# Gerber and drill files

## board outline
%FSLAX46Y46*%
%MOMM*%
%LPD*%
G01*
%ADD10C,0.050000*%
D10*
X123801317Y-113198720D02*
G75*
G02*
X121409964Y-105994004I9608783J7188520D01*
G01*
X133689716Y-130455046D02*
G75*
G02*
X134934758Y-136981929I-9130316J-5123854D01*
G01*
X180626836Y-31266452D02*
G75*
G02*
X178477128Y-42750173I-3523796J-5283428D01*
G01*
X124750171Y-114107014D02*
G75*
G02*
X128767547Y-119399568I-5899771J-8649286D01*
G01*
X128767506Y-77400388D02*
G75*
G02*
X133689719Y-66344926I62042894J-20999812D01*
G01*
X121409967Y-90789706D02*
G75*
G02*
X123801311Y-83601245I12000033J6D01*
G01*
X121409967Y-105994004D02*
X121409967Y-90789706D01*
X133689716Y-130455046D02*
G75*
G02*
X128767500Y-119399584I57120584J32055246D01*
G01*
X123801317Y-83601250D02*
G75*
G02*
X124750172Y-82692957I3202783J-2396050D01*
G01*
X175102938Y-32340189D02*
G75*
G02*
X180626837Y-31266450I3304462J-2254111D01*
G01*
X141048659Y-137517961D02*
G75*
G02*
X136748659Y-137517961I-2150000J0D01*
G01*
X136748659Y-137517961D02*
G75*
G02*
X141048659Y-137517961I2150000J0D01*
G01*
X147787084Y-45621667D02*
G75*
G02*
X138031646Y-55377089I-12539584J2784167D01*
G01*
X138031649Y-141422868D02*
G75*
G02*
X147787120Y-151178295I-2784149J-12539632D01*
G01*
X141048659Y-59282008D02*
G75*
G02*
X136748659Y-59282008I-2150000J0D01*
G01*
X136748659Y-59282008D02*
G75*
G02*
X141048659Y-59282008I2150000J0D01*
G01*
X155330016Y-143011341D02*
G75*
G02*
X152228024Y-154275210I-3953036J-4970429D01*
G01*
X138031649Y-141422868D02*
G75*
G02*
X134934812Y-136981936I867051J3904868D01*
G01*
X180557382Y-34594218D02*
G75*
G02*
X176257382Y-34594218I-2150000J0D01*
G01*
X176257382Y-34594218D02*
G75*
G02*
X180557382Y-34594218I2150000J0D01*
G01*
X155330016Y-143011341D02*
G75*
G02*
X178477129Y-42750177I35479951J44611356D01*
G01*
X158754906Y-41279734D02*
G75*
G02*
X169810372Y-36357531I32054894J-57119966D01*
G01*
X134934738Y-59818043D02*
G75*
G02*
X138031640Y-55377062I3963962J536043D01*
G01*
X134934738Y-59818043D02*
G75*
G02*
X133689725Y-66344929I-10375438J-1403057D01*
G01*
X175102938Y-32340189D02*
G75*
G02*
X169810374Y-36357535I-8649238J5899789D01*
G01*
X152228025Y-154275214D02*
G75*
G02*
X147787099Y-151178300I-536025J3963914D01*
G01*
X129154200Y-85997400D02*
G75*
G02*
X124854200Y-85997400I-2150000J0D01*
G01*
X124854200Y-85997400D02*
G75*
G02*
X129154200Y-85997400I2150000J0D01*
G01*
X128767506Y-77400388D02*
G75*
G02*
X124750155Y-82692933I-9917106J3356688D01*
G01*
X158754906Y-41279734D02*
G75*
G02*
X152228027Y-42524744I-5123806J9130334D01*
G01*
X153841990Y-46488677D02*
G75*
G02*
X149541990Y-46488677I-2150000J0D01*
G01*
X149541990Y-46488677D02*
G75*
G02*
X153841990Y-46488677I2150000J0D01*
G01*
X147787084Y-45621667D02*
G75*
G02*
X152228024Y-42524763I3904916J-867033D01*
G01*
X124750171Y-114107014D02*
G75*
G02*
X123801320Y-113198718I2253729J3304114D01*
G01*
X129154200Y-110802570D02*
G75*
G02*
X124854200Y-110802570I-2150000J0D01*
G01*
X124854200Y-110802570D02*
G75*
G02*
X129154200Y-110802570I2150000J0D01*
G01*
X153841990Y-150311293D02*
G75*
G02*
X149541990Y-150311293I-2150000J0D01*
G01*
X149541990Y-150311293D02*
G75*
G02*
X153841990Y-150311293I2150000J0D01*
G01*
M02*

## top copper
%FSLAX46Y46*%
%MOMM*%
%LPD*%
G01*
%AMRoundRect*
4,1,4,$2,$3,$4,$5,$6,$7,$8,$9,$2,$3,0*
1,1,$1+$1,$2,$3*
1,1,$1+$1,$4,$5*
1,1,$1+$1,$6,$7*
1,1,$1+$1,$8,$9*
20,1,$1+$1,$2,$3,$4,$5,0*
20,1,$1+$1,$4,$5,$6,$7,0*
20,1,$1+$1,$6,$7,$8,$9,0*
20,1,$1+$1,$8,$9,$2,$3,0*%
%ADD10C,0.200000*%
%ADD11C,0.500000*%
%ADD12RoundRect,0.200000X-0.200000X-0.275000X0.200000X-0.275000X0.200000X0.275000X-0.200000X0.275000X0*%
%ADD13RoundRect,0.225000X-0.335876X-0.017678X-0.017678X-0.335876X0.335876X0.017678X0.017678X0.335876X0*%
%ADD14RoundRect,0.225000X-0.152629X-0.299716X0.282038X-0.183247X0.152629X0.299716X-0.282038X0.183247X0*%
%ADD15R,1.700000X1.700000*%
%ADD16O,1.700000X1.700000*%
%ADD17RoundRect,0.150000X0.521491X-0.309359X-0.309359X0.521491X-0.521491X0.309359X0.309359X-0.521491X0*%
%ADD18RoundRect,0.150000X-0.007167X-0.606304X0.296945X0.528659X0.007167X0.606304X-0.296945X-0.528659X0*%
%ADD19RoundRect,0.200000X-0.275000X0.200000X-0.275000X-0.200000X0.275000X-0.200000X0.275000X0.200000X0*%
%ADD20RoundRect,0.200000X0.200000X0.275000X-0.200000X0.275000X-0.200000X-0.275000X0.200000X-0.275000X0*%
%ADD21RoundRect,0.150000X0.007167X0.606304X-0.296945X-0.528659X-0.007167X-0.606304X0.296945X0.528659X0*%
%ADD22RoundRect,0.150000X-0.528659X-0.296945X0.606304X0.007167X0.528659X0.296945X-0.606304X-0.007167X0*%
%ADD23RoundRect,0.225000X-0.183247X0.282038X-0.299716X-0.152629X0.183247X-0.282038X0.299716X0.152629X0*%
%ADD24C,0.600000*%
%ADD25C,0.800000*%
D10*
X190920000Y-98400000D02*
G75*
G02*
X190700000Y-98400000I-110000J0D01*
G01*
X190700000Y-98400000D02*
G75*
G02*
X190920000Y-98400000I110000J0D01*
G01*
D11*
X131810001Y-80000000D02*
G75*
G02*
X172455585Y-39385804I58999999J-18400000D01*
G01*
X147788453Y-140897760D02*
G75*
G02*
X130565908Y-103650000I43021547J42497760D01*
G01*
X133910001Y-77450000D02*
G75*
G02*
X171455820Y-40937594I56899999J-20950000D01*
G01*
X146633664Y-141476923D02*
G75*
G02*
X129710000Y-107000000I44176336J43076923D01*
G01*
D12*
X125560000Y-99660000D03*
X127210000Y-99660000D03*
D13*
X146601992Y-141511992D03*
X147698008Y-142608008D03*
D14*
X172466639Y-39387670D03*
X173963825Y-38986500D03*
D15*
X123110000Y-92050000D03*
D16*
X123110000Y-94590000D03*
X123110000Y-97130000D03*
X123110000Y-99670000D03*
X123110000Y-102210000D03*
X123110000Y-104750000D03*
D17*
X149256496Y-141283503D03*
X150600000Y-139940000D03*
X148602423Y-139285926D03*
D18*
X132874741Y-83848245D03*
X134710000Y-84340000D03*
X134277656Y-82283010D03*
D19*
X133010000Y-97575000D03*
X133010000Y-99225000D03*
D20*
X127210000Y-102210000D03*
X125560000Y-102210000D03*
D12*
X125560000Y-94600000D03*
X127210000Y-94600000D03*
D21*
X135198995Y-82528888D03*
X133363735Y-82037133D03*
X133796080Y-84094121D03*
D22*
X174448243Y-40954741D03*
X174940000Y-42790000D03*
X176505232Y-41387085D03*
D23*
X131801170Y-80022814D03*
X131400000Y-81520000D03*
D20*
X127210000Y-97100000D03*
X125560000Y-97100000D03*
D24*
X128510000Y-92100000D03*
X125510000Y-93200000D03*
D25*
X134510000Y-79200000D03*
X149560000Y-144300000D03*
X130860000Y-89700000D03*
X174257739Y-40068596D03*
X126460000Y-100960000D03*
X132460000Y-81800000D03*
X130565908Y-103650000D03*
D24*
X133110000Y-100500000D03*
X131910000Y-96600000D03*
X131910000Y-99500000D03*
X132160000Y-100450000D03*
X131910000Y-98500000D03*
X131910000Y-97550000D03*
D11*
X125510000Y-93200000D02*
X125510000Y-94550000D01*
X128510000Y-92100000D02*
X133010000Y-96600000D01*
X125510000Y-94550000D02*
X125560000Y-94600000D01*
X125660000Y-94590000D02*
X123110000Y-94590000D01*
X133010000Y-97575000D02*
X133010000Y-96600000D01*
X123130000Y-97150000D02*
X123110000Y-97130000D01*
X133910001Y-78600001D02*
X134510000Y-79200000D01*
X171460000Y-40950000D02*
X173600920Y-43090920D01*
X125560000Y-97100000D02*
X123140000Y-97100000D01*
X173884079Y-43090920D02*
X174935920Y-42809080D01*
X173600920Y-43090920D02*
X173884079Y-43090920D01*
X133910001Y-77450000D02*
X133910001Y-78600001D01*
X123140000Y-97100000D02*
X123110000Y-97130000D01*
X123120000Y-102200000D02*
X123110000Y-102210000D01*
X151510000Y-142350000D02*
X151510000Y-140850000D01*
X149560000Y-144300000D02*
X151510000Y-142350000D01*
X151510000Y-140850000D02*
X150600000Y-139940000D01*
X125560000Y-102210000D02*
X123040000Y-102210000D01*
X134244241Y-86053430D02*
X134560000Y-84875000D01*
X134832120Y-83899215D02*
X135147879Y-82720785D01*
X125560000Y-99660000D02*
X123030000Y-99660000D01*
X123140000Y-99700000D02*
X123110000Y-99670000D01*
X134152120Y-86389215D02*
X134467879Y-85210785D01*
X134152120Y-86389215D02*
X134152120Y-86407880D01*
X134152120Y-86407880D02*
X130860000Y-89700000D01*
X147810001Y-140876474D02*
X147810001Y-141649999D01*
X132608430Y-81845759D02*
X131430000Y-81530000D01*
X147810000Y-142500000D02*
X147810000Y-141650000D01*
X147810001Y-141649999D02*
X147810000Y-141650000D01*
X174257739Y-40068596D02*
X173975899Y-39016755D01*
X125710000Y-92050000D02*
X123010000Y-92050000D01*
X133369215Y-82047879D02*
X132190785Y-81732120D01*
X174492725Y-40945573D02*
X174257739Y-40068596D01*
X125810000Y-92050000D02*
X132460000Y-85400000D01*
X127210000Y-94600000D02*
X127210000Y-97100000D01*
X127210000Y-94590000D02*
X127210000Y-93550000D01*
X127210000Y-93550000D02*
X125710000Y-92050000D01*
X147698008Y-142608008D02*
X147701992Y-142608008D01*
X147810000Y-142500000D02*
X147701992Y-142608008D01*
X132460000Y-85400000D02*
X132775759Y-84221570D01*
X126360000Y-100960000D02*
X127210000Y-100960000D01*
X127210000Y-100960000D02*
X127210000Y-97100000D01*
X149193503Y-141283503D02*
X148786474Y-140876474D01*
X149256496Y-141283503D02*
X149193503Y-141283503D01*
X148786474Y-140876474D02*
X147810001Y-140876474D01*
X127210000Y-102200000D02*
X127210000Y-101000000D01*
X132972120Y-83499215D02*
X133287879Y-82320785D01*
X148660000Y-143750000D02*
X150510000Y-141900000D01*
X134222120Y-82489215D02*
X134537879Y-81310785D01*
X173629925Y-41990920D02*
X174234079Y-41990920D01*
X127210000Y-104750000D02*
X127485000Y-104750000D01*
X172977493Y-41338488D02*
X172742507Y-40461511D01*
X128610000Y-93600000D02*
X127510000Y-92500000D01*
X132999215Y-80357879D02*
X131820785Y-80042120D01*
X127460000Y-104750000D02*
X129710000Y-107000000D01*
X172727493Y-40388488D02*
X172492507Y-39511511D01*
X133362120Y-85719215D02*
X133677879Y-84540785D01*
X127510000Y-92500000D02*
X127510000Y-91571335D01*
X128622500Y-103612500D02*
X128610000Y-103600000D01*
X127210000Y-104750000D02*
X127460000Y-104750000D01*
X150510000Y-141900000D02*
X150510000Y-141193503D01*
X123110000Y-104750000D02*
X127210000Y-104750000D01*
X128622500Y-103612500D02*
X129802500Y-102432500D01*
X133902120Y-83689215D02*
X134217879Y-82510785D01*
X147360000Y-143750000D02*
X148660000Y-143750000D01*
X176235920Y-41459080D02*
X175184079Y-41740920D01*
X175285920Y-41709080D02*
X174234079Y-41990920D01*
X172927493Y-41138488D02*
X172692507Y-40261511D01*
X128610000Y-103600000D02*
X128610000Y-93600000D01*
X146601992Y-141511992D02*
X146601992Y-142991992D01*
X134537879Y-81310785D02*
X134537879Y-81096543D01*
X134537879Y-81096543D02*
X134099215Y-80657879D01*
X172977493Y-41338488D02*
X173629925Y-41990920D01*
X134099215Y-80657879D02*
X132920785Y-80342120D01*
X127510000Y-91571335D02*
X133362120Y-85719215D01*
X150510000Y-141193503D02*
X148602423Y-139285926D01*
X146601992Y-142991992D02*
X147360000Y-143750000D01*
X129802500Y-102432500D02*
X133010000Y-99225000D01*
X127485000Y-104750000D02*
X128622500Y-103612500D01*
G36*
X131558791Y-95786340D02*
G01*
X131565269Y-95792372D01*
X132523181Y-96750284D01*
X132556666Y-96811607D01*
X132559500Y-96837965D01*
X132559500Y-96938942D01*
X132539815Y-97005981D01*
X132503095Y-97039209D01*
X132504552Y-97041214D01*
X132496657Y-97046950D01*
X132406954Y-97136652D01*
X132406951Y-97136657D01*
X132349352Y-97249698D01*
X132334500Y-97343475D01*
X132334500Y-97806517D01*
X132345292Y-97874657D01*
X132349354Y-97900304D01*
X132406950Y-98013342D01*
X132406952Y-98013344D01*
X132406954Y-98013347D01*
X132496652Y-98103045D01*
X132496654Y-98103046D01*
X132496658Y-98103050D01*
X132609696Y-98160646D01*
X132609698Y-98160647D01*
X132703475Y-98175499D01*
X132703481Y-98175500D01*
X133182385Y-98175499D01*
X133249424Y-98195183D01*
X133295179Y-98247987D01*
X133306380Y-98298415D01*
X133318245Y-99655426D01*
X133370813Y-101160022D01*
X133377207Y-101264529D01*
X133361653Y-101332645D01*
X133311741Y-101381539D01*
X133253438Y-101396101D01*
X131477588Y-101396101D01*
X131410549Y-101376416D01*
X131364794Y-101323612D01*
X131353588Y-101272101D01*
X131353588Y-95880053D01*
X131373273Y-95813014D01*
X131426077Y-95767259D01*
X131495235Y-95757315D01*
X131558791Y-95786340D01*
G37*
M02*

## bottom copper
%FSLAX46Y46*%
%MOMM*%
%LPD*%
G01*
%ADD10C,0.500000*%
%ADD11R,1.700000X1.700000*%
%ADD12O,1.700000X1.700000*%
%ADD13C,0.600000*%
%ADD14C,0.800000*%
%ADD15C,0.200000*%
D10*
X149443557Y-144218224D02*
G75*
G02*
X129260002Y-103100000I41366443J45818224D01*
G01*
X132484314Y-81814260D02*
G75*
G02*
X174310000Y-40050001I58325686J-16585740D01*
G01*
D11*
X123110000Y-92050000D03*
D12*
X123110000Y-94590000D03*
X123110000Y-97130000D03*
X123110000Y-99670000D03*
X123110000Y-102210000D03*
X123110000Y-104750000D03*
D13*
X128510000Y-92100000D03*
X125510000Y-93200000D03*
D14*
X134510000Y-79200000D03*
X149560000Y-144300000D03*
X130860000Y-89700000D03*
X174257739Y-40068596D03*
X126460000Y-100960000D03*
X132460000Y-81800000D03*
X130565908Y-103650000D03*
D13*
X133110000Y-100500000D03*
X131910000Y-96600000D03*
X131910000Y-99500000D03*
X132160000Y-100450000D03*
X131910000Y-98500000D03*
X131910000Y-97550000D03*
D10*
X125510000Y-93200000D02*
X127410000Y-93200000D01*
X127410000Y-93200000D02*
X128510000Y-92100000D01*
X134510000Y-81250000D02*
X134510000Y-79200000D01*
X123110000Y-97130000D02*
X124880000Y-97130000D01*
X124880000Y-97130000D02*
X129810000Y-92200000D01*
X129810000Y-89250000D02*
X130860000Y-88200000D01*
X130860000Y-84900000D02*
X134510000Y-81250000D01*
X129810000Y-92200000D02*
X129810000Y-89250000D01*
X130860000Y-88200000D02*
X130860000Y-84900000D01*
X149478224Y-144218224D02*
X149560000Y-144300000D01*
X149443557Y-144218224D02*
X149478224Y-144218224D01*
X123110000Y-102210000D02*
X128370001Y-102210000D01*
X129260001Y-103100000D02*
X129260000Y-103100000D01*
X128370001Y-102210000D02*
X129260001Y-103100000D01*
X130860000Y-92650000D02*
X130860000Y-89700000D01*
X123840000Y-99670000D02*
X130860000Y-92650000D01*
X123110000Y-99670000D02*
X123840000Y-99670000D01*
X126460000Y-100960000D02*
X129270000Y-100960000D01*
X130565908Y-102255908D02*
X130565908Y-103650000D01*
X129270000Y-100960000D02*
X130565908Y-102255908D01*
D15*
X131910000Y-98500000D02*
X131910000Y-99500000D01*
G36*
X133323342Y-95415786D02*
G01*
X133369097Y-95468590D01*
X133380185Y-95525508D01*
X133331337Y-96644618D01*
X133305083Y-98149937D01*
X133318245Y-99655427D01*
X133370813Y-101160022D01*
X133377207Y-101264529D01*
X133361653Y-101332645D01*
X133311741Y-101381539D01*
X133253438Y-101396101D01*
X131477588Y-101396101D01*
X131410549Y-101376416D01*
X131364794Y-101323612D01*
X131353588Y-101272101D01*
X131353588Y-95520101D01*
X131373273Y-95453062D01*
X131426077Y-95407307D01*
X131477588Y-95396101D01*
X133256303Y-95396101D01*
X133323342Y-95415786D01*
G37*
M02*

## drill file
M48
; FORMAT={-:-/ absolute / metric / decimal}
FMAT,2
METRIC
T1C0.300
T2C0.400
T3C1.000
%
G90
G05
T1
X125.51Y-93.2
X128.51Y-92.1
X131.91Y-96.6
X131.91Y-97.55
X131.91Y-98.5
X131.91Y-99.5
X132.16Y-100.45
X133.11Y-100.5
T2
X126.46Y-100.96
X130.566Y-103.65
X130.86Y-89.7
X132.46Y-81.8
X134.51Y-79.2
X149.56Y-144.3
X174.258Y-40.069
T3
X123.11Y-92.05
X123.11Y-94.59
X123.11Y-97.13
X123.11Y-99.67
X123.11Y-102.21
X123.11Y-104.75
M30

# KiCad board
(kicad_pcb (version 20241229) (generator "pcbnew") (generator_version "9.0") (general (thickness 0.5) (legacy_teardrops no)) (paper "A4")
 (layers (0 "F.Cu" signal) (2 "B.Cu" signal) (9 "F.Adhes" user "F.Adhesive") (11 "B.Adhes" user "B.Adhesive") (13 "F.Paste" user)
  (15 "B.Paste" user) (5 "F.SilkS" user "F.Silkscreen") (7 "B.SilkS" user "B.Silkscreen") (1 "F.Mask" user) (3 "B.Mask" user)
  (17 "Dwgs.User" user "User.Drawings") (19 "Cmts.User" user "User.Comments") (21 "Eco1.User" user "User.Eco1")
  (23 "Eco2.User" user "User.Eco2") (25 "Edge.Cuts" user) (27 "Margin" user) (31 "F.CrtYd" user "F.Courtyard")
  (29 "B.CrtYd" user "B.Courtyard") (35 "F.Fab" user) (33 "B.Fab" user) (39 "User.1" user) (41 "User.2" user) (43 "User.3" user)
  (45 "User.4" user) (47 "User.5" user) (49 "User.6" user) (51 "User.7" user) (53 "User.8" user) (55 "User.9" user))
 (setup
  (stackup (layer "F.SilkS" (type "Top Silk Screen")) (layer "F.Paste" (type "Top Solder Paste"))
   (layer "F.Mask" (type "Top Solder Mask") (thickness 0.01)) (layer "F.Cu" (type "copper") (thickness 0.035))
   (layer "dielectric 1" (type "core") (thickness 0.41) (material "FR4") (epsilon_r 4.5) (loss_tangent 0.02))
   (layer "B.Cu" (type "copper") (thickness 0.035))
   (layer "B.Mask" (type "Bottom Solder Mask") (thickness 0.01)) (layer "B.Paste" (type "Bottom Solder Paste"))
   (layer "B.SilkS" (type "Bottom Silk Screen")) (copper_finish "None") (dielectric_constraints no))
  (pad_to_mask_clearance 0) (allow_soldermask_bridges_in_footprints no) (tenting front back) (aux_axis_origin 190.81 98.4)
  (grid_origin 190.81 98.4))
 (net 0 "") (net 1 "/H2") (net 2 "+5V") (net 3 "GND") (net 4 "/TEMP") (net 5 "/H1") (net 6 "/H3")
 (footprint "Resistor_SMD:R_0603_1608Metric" (layer "F.Cu") (at 126.385 99.66)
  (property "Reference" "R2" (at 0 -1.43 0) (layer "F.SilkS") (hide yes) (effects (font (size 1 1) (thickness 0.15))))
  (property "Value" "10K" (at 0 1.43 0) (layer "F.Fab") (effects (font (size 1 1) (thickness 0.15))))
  (pad "1" smd roundrect (at -0.825 0) (size 0.8 0.95) (layers "F.Cu" "F.Mask" "F.Paste") (roundrect_rratio 0.25) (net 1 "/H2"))
  (pad "2" smd roundrect (at 0.825 0) (size 0.8 0.95) (layers "F.Cu" "F.Mask" "F.Paste") (roundrect_rratio 0.25) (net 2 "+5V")))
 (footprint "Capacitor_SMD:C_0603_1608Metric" (layer "F.Cu") (at 147.15 142.06 -45)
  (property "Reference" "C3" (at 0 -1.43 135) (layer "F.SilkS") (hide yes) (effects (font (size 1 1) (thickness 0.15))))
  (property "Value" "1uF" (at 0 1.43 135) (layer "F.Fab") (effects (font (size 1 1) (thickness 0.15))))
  (pad "1" smd roundrect (at -0.775 0 315) (size 0.9 0.95) (layers "F.Cu" "F.Mask" "F.Paste") (roundrect_rratio 0.25) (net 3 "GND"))
  (pad "2" smd roundrect (at 0.775 0 315) (size 0.9 0.95) (layers "F.Cu" "F.Mask" "F.Paste") (roundrect_rratio 0.25) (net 2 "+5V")))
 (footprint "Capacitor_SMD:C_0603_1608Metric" (layer "F.Cu") (at 173.215232 39.187085 15)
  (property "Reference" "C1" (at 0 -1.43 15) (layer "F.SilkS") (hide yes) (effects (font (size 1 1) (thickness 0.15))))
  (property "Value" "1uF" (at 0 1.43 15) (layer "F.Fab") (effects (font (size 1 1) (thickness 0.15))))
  (pad "1" smd roundrect (at -0.775001 0 15) (size 0.9 0.95) (layers "F.Cu" "F.Mask" "F.Paste") (roundrect_rratio 0.25) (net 3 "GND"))
  (pad "2" smd roundrect (at 0.775001 0 15) (size 0.9 0.95) (layers "F.Cu" "F.Mask" "F.Paste") (roundrect_rratio 0.25) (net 2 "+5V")))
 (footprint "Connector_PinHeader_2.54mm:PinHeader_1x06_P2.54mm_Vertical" (layer "F.Cu") (at 123.11 92.05)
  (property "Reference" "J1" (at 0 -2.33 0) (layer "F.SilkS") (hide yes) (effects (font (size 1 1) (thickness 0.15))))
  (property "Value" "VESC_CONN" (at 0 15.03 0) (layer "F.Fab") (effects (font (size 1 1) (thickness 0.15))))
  (pad "1" thru_hole rect (at 0 0) (size 1.7 1.7) (drill 1) (layers "*.Cu" "*.Mask") (remove_unused_layers no) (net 2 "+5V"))
  (pad "2" thru_hole oval (at 0 2.54) (size 1.7 1.7) (drill 1) (layers "*.Cu" "*.Mask") (remove_unused_layers no) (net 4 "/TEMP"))
  (pad "3" thru_hole oval (at 0 5.08) (size 1.7 1.7) (drill 1) (layers "*.Cu" "*.Mask") (remove_unused_layers no) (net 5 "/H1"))
  (pad "4" thru_hole oval (at 0 7.62) (size 1.7 1.7) (drill 1) (layers "*.Cu" "*.Mask") (remove_unused_layers no) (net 1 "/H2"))
  (pad "5" thru_hole oval (at 0 10.16) (size 1.7 1.7) (drill 1) (layers "*.Cu" "*.Mask") (remove_unused_layers no) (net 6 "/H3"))
  (pad "6" thru_hole oval (at 0 12.7) (size 1.7 1.7) (drill 1) (layers "*.Cu" "*.Mask") (remove_unused_layers no) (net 3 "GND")))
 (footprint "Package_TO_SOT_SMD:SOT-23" (layer "F.Cu") (at 149.265335 139.948839 135)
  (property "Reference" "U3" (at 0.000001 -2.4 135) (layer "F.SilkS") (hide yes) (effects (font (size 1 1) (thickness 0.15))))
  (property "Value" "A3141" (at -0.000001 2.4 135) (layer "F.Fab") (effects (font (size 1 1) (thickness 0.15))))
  (pad "1" smd roundrect (at -0.9375 -0.95 135) (size 1.475 0.6) (layers "F.Cu" "F.Mask" "F.Paste") (roundrect_rratio 0.25) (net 2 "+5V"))
  (pad "2" smd roundrect (at -0.937501 0.950001 135) (size 1.475 0.6) (layers "F.Cu" "F.Mask" "F.Paste") (roundrect_rratio 0.25)
   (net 6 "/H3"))
  (pad "3" smd roundrect (at 0.9375 0.000001 135) (size 1.475 0.6) (layers "F.Cu" "F.Mask" "F.Paste") (roundrect_rratio 0.25) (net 3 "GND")))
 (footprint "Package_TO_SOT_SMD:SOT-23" (layer "F.Cu") (at 134.035013 83.188566 75)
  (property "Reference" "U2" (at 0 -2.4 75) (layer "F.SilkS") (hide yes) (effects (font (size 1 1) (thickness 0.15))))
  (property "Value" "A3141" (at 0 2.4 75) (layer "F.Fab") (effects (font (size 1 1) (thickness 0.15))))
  (pad "1" smd roundrect (at -0.937501 -0.949999 75) (size 1.475 0.6) (layers "F.Cu" "F.Mask" "F.Paste") (roundrect_rratio 0.25)
   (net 2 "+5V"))
  (pad "2" smd roundrect (at -0.9375 0.95 75) (size 1.475 0.6) (layers "F.Cu" "F.Mask" "F.Paste") (roundrect_rratio 0.25) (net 1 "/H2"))
  (pad "3" smd roundrect (at 0.937501 0 75) (size 1.475 0.6) (layers "F.Cu" "F.Mask" "F.Paste") (roundrect_rratio 0.25) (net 3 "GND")))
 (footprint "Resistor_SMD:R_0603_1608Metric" (layer "F.Cu") (at 133.01 98.4 -90)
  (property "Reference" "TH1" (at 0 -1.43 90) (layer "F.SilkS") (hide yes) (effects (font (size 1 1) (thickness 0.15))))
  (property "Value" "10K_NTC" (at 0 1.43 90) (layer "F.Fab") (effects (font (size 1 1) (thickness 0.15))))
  (pad "1" smd roundrect (at -0.825 0 270) (size 0.8 0.95) (layers "F.Cu" "F.Mask" "F.Paste") (roundrect_rratio 0.25) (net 4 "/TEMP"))
  (pad "2" smd roundrect (at 0.825 0 270) (size 0.8 0.95) (layers "F.Cu" "F.Mask" "F.Paste") (roundrect_rratio 0.25) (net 3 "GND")))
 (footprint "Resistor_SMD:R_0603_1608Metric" (layer "F.Cu") (at 126.385 102.21 180)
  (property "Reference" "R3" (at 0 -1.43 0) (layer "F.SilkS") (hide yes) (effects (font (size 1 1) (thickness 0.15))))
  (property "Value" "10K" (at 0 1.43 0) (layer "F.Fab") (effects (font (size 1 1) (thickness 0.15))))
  (pad "1" smd roundrect (at -0.825 0 180) (size 0.8 0.95) (layers "F.Cu" "F.Mask" "F.Paste") (roundrect_rratio 0.25) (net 2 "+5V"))
  (pad "2" smd roundrect (at 0.825 0 180) (size 0.8 0.95) (layers "F.Cu" "F.Mask" "F.Paste") (roundrect_rratio 0.25) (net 6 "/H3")))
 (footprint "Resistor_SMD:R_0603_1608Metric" (layer "F.Cu") (at 126.385 94.6)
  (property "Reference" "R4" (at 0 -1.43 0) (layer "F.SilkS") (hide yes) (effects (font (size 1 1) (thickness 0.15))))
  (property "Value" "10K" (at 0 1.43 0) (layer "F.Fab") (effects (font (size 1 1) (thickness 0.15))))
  (pad "1" smd roundrect (at -0.825 0) (size 0.8 0.95) (layers "F.Cu" "F.Mask" "F.Paste") (roundrect_rratio 0.25) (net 4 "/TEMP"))
  (pad "2" smd roundrect (at 0.825 0) (size 0.8 0.95) (layers "F.Cu" "F.Mask" "F.Paste") (roundrect_rratio 0.25) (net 2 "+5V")))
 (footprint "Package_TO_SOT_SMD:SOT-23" (layer "F.Cu") (at 134.038722 83.188566 -105)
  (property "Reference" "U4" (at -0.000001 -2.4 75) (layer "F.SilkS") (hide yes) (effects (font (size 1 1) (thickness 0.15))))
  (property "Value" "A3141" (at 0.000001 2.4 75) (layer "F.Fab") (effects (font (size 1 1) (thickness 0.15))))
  (pad "1" smd roundrect (at -0.937501 -0.95 255) (size 1.475 0.6) (layers "F.Cu" "F.Mask" "F.Paste") (roundrect_rratio 0.25) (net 1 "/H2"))
  (pad "2" smd roundrect (at -0.937499 0.95 255) (size 1.475 0.6) (layers "F.Cu" "F.Mask" "F.Paste") (roundrect_rratio 0.25) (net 2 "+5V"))
  (pad "3" smd roundrect (at 0.937499 -0.000001 255) (size 1.475 0.6) (layers "F.Cu" "F.Mask" "F.Paste") (roundrect_rratio 0.25)
   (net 3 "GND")))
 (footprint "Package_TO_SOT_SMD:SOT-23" (layer "F.Cu") (at 175.599677 41.629728 15)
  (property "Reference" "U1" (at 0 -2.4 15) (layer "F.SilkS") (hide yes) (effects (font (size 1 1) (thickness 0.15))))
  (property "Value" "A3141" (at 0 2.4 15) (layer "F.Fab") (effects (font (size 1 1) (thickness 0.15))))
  (pad "1" smd roundrect (at -0.9375 -0.95 15) (size 1.475 0.6) (layers "F.Cu" "F.Mask" "F.Paste") (roundrect_rratio 0.25) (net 2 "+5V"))
  (pad "2" smd roundrect (at -0.9375 0.95 15) (size 1.475 0.6) (layers "F.Cu" "F.Mask" "F.Paste") (roundrect_rratio 0.25) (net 5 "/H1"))
  (pad "3" smd roundrect (at 0.9375 0 15) (size 1.475 0.6) (layers "F.Cu" "F.Mask" "F.Paste") (roundrect_rratio 0.25) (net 3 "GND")))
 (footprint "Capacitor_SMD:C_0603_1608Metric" (layer "F.Cu") (at 131.600585 80.771407 -105)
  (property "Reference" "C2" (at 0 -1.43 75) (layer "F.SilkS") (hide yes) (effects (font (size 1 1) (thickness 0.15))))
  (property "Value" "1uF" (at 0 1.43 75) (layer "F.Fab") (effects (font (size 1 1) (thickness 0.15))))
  (pad "1" smd roundrect (at -0.775001 0 255) (size 0.9 0.95) (layers "F.Cu" "F.Mask" "F.Paste") (roundrect_rratio 0.25) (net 3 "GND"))
  (pad "2" smd roundrect (at 0.775001 0 255) (size 0.9 0.95) (layers "F.Cu" "F.Mask" "F.Paste") (roundrect_rratio 0.25) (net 2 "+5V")))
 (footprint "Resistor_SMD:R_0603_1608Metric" (layer "F.Cu") (at 126.385 97.1 180)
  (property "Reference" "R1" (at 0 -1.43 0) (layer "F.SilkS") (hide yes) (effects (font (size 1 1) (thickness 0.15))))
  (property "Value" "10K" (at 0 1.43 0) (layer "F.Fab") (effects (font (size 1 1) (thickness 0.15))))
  (pad "1" smd roundrect (at -0.825 0 180) (size 0.8 0.95) (layers "F.Cu" "F.Mask" "F.Paste") (roundrect_rratio 0.25) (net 2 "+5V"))
  (pad "2" smd roundrect (at 0.825 0 180) (size 0.8 0.95) (layers "F.Cu" "F.Mask" "F.Paste") (roundrect_rratio 0.25) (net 5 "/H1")))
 (gr_circle (center 190.81 98.4) (end 190.92 98.4) (stroke (width 0.2) (type default)) (fill no) (layer "F.Cu"))
 (gr_arc (start 131.810001 80) (mid 147.125854 54.682094) (end 172.455585 39.385804) (stroke (width 0.5) (type default)) (layer "F.Cu")
  (net 3))
 (gr_arc (start 147.788453 140.89776) (mid 135.921049 123.779444) (end 130.565908 103.65) (stroke (width 0.5) (type default)) (layer "F.Cu")
  (net 2))
 (gr_arc (start 133.910001 77.45) (mid 148.537504 54.931063) (end 171.45582 40.937595) (stroke (width 0.5) (type default)) (layer "F.Cu")
  (net 5))
 (gr_arc (start 146.633664 141.476923) (mid 135.421 125.58876) (end 129.71 107) (stroke (width 0.5) (type default)) (layer "F.Cu") (net 3))
 (gr_arc (start 149.443557 144.218224) (mid 135.396774 125.600491) (end 129.260001 103.1) (stroke (width 0.5) (type default)) (layer "B.Cu")
  (net 6))
 (gr_arc (start 132.484314 81.81426) (mid 147.963948 55.490931) (end 174.31 40.050001) (stroke (width 0.5) (type default)) (layer "B.Cu")
  (net 2))
 (gr_arc (start 123.801317 113.19872) (mid 122.020924 109.790439) (end 121.409967 105.994004) (stroke (width 0.05) (type default))
  (layer "Edge.Cuts"))
 (gr_arc (start 133.689716 130.455046) (mid 134.843739 133.617099) (end 134.934738 136.981926) (stroke (width 0.05) (type default))
  (layer "Edge.Cuts"))
 (gr_arc (start 180.626836 31.266452) (mid 183.345342 37.718415) (end 178.477129 42.750177) (stroke (width 0.05) (type default))
  (layer "Edge.Cuts"))
 (gr_arc (start 124.750171 114.107014) (mid 127.189835 116.426149) (end 128.767506 119.399582) (stroke (width 0.05) (type default))
  (layer "Edge.Cuts"))
 (gr_arc (start 128.767506 77.400388) (mid 130.972741 71.758736) (end 133.689716 66.344924) (stroke (width 0.05) (type default))
  (layer "Edge.Cuts"))
 (gr_arc (start 121.409967 90.789706) (mid 122.023488 87.001816) (end 123.801317 83.60125) (stroke (width 0.05) (type default))
  (layer "Edge.Cuts"))
 (gr_line (start 121.409967 105.994004) (end 121.409967 90.789706) (stroke (width 0.05) (type default)) (layer "Edge.Cuts"))
 (gr_arc (start 133.689716 130.455046) (mid 130.972741 125.041235) (end 128.767506 119.399582) (stroke (width 0.05) (type default))
  (layer "Edge.Cuts"))
 (gr_arc (start 123.801317 83.60125) (mid 124.238205 83.107887) (end 124.750171 82.692956) (stroke (width 0.05) (type default))
  (layer "Edge.Cuts"))
 (gr_arc (start 175.102938 32.340189) (mid 177.644145 30.667734) (end 180.626836 31.266452) (stroke (width 0.05) (type default))
  (layer "Edge.Cuts"))
 (gr_circle (center 138.898659 137.517961) (end 141.048659 137.517961) (stroke (width 0.05) (type default)) (fill no) (layer "Edge.Cuts"))
 (gr_arc (start 147.787084 45.621667) (mid 144.330246 51.920265) (end 138.031649 55.377102) (stroke (width 0.05) (type default))
  (layer "Edge.Cuts"))
 (gr_arc (start 138.031649 141.422868) (mid 144.330243 144.879709) (end 147.787084 151.178303) (stroke (width 0.05) (type default))
  (layer "Edge.Cuts"))
 (gr_circle (center 138.898659 59.282008) (end 141.048659 59.282008) (stroke (width 0.05) (type default)) (fill no) (layer "Edge.Cuts"))
 (gr_arc (start 155.330016 143.011341) (mid 157.499764 149.667944) (end 152.228025 154.275214) (stroke (width 0.05) (type default))
  (layer "Edge.Cuts"))
 (gr_arc (start 138.031649 141.422868) (mid 135.617658 139.805982) (end 134.934738 136.981926) (stroke (width 0.05) (type default))
  (layer "Edge.Cuts"))
 (gr_circle (center 178.407382 34.594218) (end 180.557382 34.594218) (stroke (width 0.05) (type default)) (fill no) (layer "Edge.Cuts"))
 (gr_arc (start 155.330016 143.011341) (mid 135.270873 85.577775) (end 178.477129 42.750177) (stroke (width 0.05) (type default))
  (layer "Edge.Cuts"))
 (gr_arc (start 158.754906 41.279734) (mid 164.168716 38.562756) (end 169.81037 36.357524) (stroke (width 0.05) (type default))
  (layer "Edge.Cuts"))
 (gr_arc (start 134.934738 59.818043) (mid 135.61766 56.99399) (end 138.031649 55.377102) (stroke (width 0.05) (type default))
  (layer "Edge.Cuts"))
 (gr_arc (start 134.934738 59.818043) (mid 134.843738 63.182871) (end 133.689716 66.344924) (stroke (width 0.05) (type default))
  (layer "Edge.Cuts"))
 (gr_arc (start 175.102938 32.340189) (mid 172.783804 34.779856) (end 169.81037 36.357524) (stroke (width 0.05) (type default))
  (layer "Edge.Cuts"))
 (gr_arc (start 152.228025 154.275214) (mid 149.403967 153.592295) (end 147.787084 151.178303) (stroke (width 0.05) (type default))
  (layer "Edge.Cuts"))
 (gr_circle (center 127.0042 85.9974) (end 129.1542 85.9974) (stroke (width 0.05) (type default)) (fill no) (layer "Edge.Cuts"))
 (gr_arc (start 128.767506 77.400388) (mid 127.189835 80.373821) (end 124.750171 82.692956) (stroke (width 0.05) (type default))
  (layer "Edge.Cuts"))
 (gr_arc (start 158.754906 41.279734) (mid 155.592853 42.433758) (end 152.228025 42.524756) (stroke (width 0.05) (type default))
  (layer "Edge.Cuts"))
 (gr_circle (center 151.69199 46.488677) (end 153.84199 46.488677) (stroke (width 0.05) (type default)) (fill no) (layer "Edge.Cuts"))
 (gr_arc (start 147.787084 45.621667) (mid 149.403971 43.207681) (end 152.228025 42.524756) (stroke (width 0.05) (type default))
  (layer "Edge.Cuts"))
 (gr_arc (start 124.750171 114.107014) (mid 124.238202 113.692085) (end 123.801317 113.19872) (stroke (width 0.05) (type default))
  (layer "Edge.Cuts"))
 (gr_circle (center 127.0042 110.80257) (end 129.1542 110.80257) (stroke (width 0.05) (type default)) (fill no) (layer "Edge.Cuts"))
 (gr_circle (center 151.69199 150.311293) (end 153.84199 150.311293) (stroke (width 0.05) (type default)) (fill no) (layer "Edge.Cuts"))
 (segment (start 125.51 93.2) (end 125.51 94.55) (width 0.5) (layer "F.Cu") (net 4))
 (segment (start 128.51 92.1) (end 133.01 96.6) (width 0.5) (layer "F.Cu") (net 4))
 (segment (start 125.51 94.55) (end 125.56 94.6) (width 0.5) (layer "F.Cu") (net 4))
 (segment (start 125.66 94.59) (end 123.11 94.59) (width 0.5) (layer "F.Cu") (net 4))
 (segment (start 133.01 97.575) (end 133.01 96.6) (width 0.5) (layer "F.Cu") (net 4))
 (via (at 128.51 92.1) (size 0.6) (drill 0.3) (layers "F.Cu" "B.Cu") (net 4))
 (via (at 125.51 93.2) (size 0.6) (drill 0.3) (layers "F.Cu" "B.Cu") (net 4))
 (segment (start 125.51 93.2) (end 127.41 93.2) (width 0.5) (layer "B.Cu") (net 4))
 (segment (start 127.41 93.2) (end 128.51 92.1) (width 0.5) (layer "B.Cu") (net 4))
 (segment (start 123.13 97.15) (end 123.11 97.13) (width 0.5) (layer "F.Cu") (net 5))
 (segment (start 133.910001 78.600001) (end 134.51 79.2) (width 0.5) (layer "F.Cu") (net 5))
 (segment (start 171.46 40.95) (end 173.60092 43.09092) (width 0.5) (layer "F.Cu") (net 5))
 (segment (start 125.56 97.1) (end 123.14 97.1) (width 0.5) (layer "F.Cu") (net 5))
 (segment (start 173.884079 43.09092) (end 174.93592 42.80908) (width 0.5) (layer "F.Cu") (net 5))
 (segment (start 173.60092 43.09092) (end 173.884079 43.09092) (width 0.5) (layer "F.Cu") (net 5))
 (segment (start 133.910001 77.45) (end 133.910001 78.600001) (width 0.5) (layer "F.Cu") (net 5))
 (segment (start 123.14 97.1) (end 123.11 97.13) (width 0.5) (layer "F.Cu") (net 5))
 (via (at 134.51 79.2) (size 0.8) (drill 0.4) (layers "F.Cu" "B.Cu") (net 5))
 (segment (start 134.51 81.25) (end 134.51 79.2) (width 0.5) (layer "B.Cu") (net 5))
 (segment (start 123.11 97.13) (end 124.88 97.13) (width 0.5) (layer "B.Cu") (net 5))
 (segment (start 124.88 97.13) (end 129.81 92.2) (width 0.5) (layer "B.Cu") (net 5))
 (segment (start 129.81 89.25) (end 130.86 88.2) (width 0.5) (layer "B.Cu") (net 5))
 (segment (start 130.86 84.9) (end 134.51 81.25) (width 0.5) (layer "B.Cu") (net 5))
 (segment (start 129.81 92.2) (end 129.81 89.25) (width 0.5) (layer "B.Cu") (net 5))
 (segment (start 130.86 88.2) (end 130.86 84.9) (width 0.5) (layer "B.Cu") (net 5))
 (segment (start 123.12 102.2) (end 123.11 102.21) (width 0.5) (layer "F.Cu") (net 6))
 (segment (start 151.51 142.35) (end 151.51 140.85) (width 0.5) (layer "F.Cu") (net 6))
 (segment (start 149.56 144.3) (end 151.51 142.35) (width 0.5) (layer "F.Cu") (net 6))
 (segment (start 151.51 140.85) (end 150.6 139.94) (width 0.5) (layer "F.Cu") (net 6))
 (segment (start 125.56 102.21) (end 123.04 102.21) (width 0.5) (layer "F.Cu") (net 6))
 (via (at 149.56 144.3) (size 0.8) (drill 0.4) (layers "F.Cu" "B.Cu") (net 6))
 (segment (start 149.478224 144.218224) (end 149.56 144.3) (width 0.5) (layer "B.Cu") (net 6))
 (segment (start 149.443557 144.218224) (end 149.478224 144.218224) (width 0.5) (layer "B.Cu") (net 6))
 (segment (start 123.11 102.21) (end 128.370001 102.21) (width 0.5) (layer "B.Cu") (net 6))
 (segment (start 129.260001 103.1) (end 129.26 103.1) (width 0.5) (layer "B.Cu") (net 6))
 (segment (start 128.370001 102.21) (end 129.260001 103.1) (width 0.5) (layer "B.Cu") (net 6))
 (segment (start 134.244241 86.05343) (end 134.56 84.875) (width 0.5) (layer "F.Cu") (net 1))
 (segment (start 134.83212 83.899215) (end 135.147879 82.720785) (width 0.5) (layer "F.Cu") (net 1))
 (segment (start 125.56 99.66) (end 123.03 99.66) (width 0.5) (layer "F.Cu") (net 1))
 (segment (start 123.14 99.7) (end 123.11 99.67) (width 0.5) (layer "F.Cu") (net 1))
 (segment (start 134.15212 86.389215) (end 134.467879 85.210785) (width 0.5) (layer "F.Cu") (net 1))
 (segment (start 134.15212 86.389215) (end 134.15212 86.40788) (width 0.5) (layer "F.Cu") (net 1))
 (segment (start 134.15212 86.40788) (end 130.86 89.7) (width 0.5) (layer "F.Cu") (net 1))
 (via (at 130.86 89.7) (size 0.8) (drill 0.4) (layers "F.Cu" "B.Cu") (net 1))
 (segment (start 130.86 92.65) (end 130.86 89.7) (width 0.5) (layer "B.Cu") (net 1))
 (segment (start 123.84 99.67) (end 130.86 92.65) (width 0.5) (layer "B.Cu") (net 1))
 (segment (start 123.11 99.67) (end 123.84 99.67) (width 0.5) (layer "B.Cu") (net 1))
 (segment (start 147.810001 140.876474) (end 147.810001 141.649999) (width 0.5) (layer "F.Cu") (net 2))
 (segment (start 132.60843 81.845759) (end 131.43 81.53) (width 0.5) (layer "F.Cu") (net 2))
 (segment (start 147.81 142.5) (end 147.81 141.65) (width 0.5) (layer "F.Cu") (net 2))
 (segment (start 147.810001 141.649999) (end 147.81 141.65) (width 0.5) (layer "F.Cu") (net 2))
 (segment (start 174.257739 40.068596) (end 173.975899 39.016755) (width 0.5) (layer "F.Cu") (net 2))
 (segment (start 125.71 92.05) (end 123.01 92.05) (width 0.5) (layer "F.Cu") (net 2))
 (segment (start 133.369215 82.047879) (end 132.190785 81.73212) (width 0.5) (layer "F.Cu") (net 2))
 (segment (start 174.492725 40.945573) (end 174.257739 40.068596) (width 0.5) (layer "F.Cu") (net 2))
 (segment (start 125.81 92.05) (end 132.46 85.4) (width 0.5) (layer "F.Cu") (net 2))
 (segment (start 127.21 94.6) (end 127.21 97.1) (width 0.5) (layer "F.Cu") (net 2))
 (segment (start 127.21 94.59) (end 127.21 93.55) (width 0.5) (layer "F.Cu") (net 2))
 (segment (start 127.21 93.55) (end 125.71 92.05) (width 0.5) (layer "F.Cu") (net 2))
 (segment (start 147.698008 142.608008) (end 147.701992 142.608008) (width 0.5) (layer "F.Cu") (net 2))
 (segment (start 147.81 142.5) (end 147.701992 142.608008) (width 0.5) (layer "F.Cu") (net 2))
 (segment (start 132.46 85.4) (end 132.775759 84.22157) (width 0.5) (layer "F.Cu") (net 2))
 (segment (start 126.36 100.96) (end 127.21 100.96) (width 0.5) (layer "F.Cu") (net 2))
 (segment (start 127.21 100.96) (end 127.21 97.1) (width 0.5) (layer "F.Cu") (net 2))
 (segment (start 149.193503 141.283503) (end 148.786474 140.876474) (width 0.5) (layer "F.Cu") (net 2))
 (segment (start 149.256496 141.283503) (end 149.193503 141.283503) (width 0.5) (layer "F.Cu") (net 2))
 (segment (start 148.786474 140.876474) (end 147.810001 140.876474) (width 0.5) (layer "F.Cu") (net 2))
 (segment (start 127.21 102.2) (end 127.21 101) (width 0.5) (layer "F.Cu") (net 2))
 (segment (start 132.97212 83.499215) (end 133.287879 82.320785) (width 0.5) (layer "F.Cu") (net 2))
 (via (at 174.257739 40.068596) (size 0.8) (drill 0.4) (layers "F.Cu" "B.Cu") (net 2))
 (via (at 126.46 100.96) (size 0.8) (drill 0.4) (layers "F.Cu" "B.Cu") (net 2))
 (via (at 132.46 81.8) (size 0.8) (drill 0.4) (layers "F.Cu" "B.Cu") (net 2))
 (via (at 130.565908 103.65) (size 0.8) (drill 0.4) (layers "F.Cu" "B.Cu") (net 2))
 (segment (start 126.46 100.96) (end 129.27 100.96) (width 0.5) (layer "B.Cu") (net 2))
 (segment (start 130.565908 102.255908) (end 130.565908 103.65) (width 0.5) (layer "B.Cu") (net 2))
 (segment (start 129.27 100.96) (end 130.565908 102.255908) (width 0.5) (layer "B.Cu") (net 2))
 (segment (start 148.66 143.75) (end 150.51 141.9) (width 0.5) (layer "F.Cu") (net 3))
 (segment (start 134.22212 82.489215) (end 134.537879 81.310785) (width 0.5) (layer "F.Cu") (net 3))
 (segment (start 173.629925 41.99092) (end 174.234079 41.99092) (width 0.5) (layer "F.Cu") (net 3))
 (segment (start 127.21 104.75) (end 127.485 104.75) (width 0.5) (layer "F.Cu") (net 3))
 (segment (start 172.977493 41.338488) (end 172.742507 40.461511) (width 0.5) (layer "F.Cu") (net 3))
 (segment (start 128.61 93.6) (end 127.51 92.5) (width 0.5) (layer "F.Cu") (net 3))
 (segment (start 132.999215 80.357879) (end 131.820785 80.04212) (width 0.5) (layer "F.Cu") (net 3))
 (segment (start 127.46 104.75) (end 129.71 107) (width 0.5) (layer "F.Cu") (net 3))
 (segment (start 172.727493 40.388488) (end 172.492507 39.511511) (width 0.5) (layer "F.Cu") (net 3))
 (segment (start 133.36212 85.719215) (end 133.677879 84.540785) (width 0.5) (layer "F.Cu") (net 3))
 (segment (start 127.51 92.5) (end 127.51 91.571335) (width 0.5) (layer "F.Cu") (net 3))
 (segment (start 128.6225 103.6125) (end 128.61 103.6) (width 0.5) (layer "F.Cu") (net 3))
 (segment (start 127.21 104.75) (end 127.46 104.75) (width 0.5) (layer "F.Cu") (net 3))
 (segment (start 150.51 141.9) (end 150.51 141.193503) (width 0.5) (layer "F.Cu") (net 3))
 (segment (start 123.11 104.75) (end 127.21 104.75) (width 0.5) (layer "F.Cu") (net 3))
 (segment (start 128.6225 103.6125) (end 129.8025 102.4325) (width 0.5) (layer "F.Cu") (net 3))
 (segment (start 133.90212 83.689215) (end 134.217879 82.510785) (width 0.5) (layer "F.Cu") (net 3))
 (segment (start 147.36 143.75) (end 148.66 143.75) (width 0.5) (layer "F.Cu") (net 3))
 (segment (start 176.23592 41.45908) (end 175.184079 41.74092) (width 0.5) (layer "F.Cu") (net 3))
 (segment (start 175.28592 41.70908) (end 174.234079 41.99092) (width 0.5) (layer "F.Cu") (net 3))
 (segment (start 172.927493 41.138488) (end 172.692507 40.261511) (width 0.5) (layer "F.Cu") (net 3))
 (segment (start 128.61 103.6) (end 128.61 93.6) (width 0.5) (layer "F.Cu") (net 3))
 (segment (start 146.601992 141.511992) (end 146.601992 142.991992) (width 0.5) (layer "F.Cu") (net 3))
 (segment (start 134.537879 81.310785) (end 134.537879 81.096543) (width 0.5) (layer "F.Cu") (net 3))
 (segment (start 134.537879 81.096543) (end 134.099215 80.657879) (width 0.5) (layer "F.Cu") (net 3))
 (segment (start 172.977493 41.338488) (end 173.629925 41.99092) (width 0.5) (layer "F.Cu") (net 3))
 (segment (start 134.099215 80.657879) (end 132.920785 80.34212) (width 0.5) (layer "F.Cu") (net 3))
 (segment (start 127.51 91.571335) (end 133.36212 85.719215) (width 0.5) (layer "F.Cu") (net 3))
 (segment (start 150.51 141.193503) (end 148.602423 139.285926) (width 0.5) (layer "F.Cu") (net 3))
 (segment (start 146.601992 142.991992) (end 147.36 143.75) (width 0.5) (layer "F.Cu") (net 3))
 (segment (start 129.8025 102.4325) (end 133.01 99.225) (width 0.5) (layer "F.Cu") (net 3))
 (segment (start 127.485 104.75) (end 128.6225 103.6125) (width 0.5) (layer "F.Cu") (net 3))
 (via (at 133.11 100.5) (size 0.6) (drill 0.3) (layers "F.Cu" "B.Cu") (free yes) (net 3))
 (via (at 131.91 96.6) (size 0.6) (drill 0.3) (layers "F.Cu" "B.Cu") (free yes) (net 3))
 (via (at 131.91 99.5) (size 0.6) (drill 0.3) (layers "F.Cu" "B.Cu") (free yes) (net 3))
 (via (at 132.16 100.45) (size 0.6) (drill 0.3) (layers "F.Cu" "B.Cu") (free yes) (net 3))
 (via (at 131.91 98.5) (size 0.6) (drill 0.3) (layers "F.Cu" "B.Cu") (free yes) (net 3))
 (via (at 131.91 97.55) (size 0.6) (drill 0.3) (layers "F.Cu" "B.Cu") (free yes) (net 3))
 (segment (start 131.91 98.5) (end 131.91 99.5) (width 0.2) (layer "B.Cu") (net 3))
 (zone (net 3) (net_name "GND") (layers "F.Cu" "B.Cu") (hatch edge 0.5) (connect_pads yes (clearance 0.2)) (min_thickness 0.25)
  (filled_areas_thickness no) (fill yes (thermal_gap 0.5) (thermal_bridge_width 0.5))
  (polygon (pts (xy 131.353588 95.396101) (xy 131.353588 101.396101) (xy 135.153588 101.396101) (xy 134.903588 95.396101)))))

